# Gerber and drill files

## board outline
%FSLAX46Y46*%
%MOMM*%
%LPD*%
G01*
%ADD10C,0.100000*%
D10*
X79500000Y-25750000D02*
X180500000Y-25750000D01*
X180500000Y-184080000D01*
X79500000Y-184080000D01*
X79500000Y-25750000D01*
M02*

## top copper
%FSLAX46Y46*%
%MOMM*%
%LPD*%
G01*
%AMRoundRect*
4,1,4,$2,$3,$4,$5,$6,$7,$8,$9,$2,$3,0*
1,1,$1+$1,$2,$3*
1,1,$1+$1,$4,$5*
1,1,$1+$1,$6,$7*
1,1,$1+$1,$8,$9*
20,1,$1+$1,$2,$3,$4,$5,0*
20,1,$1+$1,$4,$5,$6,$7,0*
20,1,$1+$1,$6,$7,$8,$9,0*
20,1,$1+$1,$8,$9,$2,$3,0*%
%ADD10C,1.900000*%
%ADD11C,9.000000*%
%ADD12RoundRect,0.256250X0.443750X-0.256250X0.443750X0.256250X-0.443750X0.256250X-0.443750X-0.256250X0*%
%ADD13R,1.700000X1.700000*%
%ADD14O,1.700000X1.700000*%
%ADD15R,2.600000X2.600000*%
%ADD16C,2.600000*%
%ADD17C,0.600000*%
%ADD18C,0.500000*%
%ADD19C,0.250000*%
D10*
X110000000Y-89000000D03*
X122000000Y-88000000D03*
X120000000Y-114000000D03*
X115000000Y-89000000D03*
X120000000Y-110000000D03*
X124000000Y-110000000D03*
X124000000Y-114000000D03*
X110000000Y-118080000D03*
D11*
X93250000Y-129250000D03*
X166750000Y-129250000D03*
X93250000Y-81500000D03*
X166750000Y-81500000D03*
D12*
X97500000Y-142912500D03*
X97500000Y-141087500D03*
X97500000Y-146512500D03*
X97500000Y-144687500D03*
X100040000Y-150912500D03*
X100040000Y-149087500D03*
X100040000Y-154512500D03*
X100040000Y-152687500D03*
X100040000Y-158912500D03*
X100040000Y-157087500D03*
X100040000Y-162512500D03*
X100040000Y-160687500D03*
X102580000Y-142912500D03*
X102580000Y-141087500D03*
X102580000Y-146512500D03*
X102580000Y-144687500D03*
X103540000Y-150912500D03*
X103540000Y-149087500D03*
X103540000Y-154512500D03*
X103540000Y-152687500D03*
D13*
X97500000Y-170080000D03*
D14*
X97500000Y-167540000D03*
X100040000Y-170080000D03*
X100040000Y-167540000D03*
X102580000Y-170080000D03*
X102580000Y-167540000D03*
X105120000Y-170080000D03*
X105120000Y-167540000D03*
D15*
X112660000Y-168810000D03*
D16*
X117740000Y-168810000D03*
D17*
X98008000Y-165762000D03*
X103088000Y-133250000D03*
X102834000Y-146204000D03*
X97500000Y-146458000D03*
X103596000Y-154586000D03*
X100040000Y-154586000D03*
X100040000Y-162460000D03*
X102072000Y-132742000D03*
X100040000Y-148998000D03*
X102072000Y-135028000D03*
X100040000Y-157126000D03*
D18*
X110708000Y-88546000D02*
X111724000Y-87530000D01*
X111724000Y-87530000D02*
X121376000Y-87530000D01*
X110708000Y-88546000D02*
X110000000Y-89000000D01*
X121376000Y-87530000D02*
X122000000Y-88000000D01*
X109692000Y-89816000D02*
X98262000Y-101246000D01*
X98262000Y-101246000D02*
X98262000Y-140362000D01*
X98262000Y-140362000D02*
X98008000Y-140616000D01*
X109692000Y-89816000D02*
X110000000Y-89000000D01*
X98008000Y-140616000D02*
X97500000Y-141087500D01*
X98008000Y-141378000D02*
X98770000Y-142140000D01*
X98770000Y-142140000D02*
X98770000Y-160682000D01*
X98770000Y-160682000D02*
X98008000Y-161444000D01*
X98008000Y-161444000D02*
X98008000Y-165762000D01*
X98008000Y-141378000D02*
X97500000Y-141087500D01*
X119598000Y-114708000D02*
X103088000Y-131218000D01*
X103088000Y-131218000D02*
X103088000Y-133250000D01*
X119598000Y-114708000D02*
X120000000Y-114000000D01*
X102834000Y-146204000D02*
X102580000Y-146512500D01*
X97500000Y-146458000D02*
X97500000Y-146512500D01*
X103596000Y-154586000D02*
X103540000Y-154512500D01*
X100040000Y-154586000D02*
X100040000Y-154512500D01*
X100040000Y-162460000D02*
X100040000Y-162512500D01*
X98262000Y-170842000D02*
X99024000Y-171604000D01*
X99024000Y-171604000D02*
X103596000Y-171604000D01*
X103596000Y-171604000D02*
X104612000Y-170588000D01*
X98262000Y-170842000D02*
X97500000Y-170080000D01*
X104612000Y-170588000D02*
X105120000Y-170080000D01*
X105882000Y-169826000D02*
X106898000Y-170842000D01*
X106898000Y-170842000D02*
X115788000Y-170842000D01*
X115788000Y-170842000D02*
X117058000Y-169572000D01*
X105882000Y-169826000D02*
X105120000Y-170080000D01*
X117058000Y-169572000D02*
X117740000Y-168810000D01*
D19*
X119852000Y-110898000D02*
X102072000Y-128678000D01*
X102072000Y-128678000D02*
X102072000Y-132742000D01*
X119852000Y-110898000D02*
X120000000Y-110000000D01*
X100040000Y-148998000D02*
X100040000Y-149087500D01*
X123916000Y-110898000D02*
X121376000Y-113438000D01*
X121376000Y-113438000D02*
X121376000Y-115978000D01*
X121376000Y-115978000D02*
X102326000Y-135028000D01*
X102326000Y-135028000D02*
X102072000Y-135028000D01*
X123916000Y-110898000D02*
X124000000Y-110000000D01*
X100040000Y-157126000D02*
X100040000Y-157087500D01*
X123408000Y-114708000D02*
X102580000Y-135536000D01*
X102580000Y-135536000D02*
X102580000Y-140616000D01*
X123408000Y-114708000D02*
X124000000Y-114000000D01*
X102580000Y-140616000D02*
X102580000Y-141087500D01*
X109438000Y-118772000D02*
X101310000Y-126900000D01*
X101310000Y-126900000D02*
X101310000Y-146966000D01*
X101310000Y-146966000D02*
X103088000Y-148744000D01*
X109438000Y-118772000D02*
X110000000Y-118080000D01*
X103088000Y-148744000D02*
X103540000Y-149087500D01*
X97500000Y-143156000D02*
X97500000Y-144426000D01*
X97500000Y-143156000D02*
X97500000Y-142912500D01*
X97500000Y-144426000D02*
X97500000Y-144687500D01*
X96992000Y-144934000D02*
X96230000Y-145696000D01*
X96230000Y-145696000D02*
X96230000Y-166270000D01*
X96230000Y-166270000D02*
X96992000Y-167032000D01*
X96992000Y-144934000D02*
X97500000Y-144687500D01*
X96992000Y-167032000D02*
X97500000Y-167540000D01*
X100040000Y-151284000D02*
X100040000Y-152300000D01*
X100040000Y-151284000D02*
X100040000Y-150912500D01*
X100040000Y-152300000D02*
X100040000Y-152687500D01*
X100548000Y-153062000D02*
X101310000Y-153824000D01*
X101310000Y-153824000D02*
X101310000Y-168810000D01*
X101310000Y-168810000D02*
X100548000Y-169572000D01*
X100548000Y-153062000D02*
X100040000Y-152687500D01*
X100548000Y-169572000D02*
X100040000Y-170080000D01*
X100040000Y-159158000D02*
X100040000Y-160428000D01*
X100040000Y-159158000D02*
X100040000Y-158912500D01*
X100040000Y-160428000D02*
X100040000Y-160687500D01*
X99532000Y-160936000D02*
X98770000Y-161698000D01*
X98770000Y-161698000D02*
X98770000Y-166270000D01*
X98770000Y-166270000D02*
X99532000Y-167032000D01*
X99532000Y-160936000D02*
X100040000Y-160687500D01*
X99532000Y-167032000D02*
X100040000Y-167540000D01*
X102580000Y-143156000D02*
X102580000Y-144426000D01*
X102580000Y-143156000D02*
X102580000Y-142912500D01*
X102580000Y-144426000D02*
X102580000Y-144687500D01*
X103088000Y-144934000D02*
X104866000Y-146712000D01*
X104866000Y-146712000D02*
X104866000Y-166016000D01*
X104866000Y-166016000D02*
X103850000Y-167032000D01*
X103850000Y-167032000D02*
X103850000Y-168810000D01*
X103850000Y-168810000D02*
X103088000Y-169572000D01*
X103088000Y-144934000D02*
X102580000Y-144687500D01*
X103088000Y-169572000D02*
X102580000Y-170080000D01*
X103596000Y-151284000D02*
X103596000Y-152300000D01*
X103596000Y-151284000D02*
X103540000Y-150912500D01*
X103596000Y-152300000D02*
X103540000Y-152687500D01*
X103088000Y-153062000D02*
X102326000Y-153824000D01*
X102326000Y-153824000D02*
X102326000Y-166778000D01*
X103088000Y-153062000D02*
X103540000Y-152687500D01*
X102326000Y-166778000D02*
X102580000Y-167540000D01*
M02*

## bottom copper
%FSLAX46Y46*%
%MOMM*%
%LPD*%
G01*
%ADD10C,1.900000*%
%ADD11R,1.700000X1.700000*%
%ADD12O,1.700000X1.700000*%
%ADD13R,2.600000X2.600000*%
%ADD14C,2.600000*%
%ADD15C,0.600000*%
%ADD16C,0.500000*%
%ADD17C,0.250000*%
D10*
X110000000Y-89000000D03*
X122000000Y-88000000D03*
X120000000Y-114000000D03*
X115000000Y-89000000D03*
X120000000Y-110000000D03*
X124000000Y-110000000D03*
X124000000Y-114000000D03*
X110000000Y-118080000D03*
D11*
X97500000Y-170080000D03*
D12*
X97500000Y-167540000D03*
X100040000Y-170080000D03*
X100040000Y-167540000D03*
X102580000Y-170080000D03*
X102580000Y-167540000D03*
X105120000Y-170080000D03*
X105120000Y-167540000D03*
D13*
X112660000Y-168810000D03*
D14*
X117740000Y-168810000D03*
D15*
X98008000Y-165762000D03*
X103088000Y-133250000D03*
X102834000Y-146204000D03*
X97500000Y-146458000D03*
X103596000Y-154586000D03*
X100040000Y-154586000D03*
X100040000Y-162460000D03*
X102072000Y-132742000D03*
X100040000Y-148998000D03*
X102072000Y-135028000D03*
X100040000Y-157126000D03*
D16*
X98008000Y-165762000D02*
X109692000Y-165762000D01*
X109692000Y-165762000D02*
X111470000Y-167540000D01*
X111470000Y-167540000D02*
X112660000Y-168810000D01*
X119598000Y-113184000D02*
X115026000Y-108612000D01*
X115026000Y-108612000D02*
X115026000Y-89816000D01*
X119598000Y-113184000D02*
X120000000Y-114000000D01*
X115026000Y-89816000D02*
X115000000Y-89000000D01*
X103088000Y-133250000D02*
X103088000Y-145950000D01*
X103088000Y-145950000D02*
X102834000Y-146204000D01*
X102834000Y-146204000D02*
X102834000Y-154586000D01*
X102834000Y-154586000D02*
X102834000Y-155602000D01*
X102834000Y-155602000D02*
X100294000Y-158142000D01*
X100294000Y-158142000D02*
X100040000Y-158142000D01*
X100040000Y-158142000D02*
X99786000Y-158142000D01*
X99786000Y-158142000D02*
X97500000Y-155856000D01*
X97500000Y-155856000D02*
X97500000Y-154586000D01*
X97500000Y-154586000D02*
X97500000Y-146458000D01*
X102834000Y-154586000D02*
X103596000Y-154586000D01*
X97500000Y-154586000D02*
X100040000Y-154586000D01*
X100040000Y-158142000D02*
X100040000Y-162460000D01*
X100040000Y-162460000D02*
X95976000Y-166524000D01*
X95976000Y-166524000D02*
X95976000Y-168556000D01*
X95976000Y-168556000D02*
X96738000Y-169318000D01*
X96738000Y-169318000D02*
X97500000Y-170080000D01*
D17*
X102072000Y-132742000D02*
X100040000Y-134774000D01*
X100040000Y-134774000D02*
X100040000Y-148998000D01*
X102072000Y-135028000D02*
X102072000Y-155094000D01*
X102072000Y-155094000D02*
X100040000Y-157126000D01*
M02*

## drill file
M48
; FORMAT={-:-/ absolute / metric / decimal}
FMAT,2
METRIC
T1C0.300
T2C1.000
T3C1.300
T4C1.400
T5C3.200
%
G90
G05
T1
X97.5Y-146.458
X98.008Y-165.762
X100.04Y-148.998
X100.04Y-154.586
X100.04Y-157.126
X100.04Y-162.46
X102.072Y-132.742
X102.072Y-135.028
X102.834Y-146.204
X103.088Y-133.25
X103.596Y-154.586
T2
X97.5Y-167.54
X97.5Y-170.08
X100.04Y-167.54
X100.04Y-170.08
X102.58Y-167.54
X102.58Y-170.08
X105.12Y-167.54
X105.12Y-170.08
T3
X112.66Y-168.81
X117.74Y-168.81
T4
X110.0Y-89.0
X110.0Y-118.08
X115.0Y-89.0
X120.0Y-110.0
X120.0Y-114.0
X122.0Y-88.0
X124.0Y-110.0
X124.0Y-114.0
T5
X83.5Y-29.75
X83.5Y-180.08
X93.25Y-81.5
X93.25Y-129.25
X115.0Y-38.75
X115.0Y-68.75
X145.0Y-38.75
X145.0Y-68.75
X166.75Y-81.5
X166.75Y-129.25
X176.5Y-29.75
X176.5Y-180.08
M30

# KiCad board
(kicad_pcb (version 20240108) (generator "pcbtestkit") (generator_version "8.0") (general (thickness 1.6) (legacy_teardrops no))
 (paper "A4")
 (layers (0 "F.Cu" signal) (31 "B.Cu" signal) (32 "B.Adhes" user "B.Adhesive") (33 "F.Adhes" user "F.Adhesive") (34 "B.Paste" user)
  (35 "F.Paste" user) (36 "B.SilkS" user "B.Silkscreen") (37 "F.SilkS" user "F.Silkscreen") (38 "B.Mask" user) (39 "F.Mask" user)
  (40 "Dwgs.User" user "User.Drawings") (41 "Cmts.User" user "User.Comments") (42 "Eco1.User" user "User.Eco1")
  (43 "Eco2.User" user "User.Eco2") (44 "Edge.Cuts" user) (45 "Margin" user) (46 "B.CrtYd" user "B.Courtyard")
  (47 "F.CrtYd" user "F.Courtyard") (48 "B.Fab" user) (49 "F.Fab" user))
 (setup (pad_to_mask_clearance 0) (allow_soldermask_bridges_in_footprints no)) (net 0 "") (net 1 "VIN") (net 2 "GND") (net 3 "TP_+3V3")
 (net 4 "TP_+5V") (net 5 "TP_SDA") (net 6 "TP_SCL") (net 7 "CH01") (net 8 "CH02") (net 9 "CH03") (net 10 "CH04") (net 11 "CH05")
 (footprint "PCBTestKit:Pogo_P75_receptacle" (layer "F.Cu") (at 110 89)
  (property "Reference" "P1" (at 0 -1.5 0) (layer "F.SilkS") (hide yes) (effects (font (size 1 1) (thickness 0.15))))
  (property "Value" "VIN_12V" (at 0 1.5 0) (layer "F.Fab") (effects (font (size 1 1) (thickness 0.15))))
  (pad "1" thru_hole circle (at 0 0) (size 1.9 1.9) (drill 1.4) (layers "*.Cu" "*.Mask") (remove_unused_layers no) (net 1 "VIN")))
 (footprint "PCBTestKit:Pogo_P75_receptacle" (layer "F.Cu") (at 122 88)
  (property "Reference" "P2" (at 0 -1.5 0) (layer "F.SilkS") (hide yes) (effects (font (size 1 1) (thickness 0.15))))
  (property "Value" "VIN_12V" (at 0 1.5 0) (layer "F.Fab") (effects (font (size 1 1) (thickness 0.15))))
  (pad "1" thru_hole circle (at 0 0) (size 1.9 1.9) (drill 1.4) (layers "*.Cu" "*.Mask") (remove_unused_layers no) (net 1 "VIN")))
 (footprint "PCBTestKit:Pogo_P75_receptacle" (layer "F.Cu") (at 120 114)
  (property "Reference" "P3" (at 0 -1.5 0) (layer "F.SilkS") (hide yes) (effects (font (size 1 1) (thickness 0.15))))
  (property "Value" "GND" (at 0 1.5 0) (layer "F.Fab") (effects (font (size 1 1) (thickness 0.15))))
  (pad "1" thru_hole circle (at 0 0) (size 1.9 1.9) (drill 1.4) (layers "*.Cu" "*.Mask") (remove_unused_layers no) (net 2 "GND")))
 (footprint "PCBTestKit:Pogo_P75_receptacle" (layer "F.Cu") (at 115 89)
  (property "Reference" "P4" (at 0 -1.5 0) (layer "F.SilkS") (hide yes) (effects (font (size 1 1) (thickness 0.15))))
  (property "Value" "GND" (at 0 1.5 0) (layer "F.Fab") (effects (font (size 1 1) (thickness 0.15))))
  (pad "1" thru_hole circle (at 0 0) (size 1.9 1.9) (drill 1.4) (layers "*.Cu" "*.Mask") (remove_unused_layers no) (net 2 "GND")))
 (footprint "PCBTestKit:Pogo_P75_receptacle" (layer "F.Cu") (at 120 110)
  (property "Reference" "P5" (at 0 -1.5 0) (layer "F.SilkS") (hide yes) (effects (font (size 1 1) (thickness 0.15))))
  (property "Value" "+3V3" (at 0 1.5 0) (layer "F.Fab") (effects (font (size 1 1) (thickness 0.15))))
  (pad "1" thru_hole circle (at 0 0) (size 1.9 1.9) (drill 1.4) (layers "*.Cu" "*.Mask") (remove_unused_layers no) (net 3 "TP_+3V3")))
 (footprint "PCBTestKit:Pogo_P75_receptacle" (layer "F.Cu") (at 124 110)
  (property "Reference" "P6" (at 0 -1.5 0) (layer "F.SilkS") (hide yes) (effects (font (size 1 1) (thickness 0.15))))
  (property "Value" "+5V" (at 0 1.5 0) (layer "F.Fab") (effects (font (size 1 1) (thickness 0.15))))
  (pad "1" thru_hole circle (at 0 0) (size 1.9 1.9) (drill 1.4) (layers "*.Cu" "*.Mask") (remove_unused_layers no) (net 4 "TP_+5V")))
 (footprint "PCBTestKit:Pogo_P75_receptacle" (layer "F.Cu") (at 124 114)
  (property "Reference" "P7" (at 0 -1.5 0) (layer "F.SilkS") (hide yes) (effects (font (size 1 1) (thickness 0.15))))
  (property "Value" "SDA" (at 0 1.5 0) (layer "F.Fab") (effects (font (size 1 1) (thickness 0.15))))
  (pad "1" thru_hole circle (at 0 0) (size 1.9 1.9) (drill 1.4) (layers "*.Cu" "*.Mask") (remove_unused_layers no) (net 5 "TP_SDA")))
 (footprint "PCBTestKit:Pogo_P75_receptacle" (layer "F.Cu") (at 110 118.08)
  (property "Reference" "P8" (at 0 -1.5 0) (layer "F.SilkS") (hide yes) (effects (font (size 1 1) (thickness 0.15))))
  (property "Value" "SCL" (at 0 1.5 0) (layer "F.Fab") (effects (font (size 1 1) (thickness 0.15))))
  (pad "1" thru_hole circle (at 0 0) (size 1.9 1.9) (drill 1.4) (layers "*.Cu" "*.Mask") (remove_unused_layers no) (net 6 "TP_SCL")))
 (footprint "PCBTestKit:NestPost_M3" (layer "F.Cu") (at 93.25 129.25)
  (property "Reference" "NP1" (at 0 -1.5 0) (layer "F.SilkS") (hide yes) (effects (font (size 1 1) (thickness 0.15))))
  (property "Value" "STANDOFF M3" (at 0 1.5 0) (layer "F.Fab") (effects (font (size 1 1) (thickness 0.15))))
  (pad "" np_thru_hole circle (at 0 0) (size 9 9) (drill 3.2) (layers "F.Cu" "F.Mask")))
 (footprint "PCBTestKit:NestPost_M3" (layer "F.Cu") (at 166.75 129.25)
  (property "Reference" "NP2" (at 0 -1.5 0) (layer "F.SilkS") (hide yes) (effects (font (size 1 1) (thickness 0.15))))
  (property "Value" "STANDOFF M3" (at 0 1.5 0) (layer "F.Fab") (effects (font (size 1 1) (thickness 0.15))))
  (pad "" np_thru_hole circle (at 0 0) (size 9 9) (drill 3.2) (layers "F.Cu" "F.Mask")))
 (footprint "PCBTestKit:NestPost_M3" (layer "F.Cu") (at 93.25 81.5)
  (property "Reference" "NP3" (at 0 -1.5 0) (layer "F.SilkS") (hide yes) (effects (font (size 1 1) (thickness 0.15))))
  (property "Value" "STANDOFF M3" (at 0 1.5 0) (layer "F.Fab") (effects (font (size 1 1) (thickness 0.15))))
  (pad "" np_thru_hole circle (at 0 0) (size 9 9) (drill 3.2) (layers "F.Cu" "F.Mask")))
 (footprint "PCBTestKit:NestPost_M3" (layer "F.Cu") (at 166.75 81.5)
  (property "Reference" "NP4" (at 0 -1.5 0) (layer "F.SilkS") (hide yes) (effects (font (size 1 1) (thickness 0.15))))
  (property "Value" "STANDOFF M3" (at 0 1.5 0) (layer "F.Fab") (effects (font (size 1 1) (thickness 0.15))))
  (pad "" np_thru_hole circle (at 0 0) (size 9 9) (drill 3.2) (layers "F.Cu" "F.Mask")))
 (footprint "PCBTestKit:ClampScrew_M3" (layer "F.Cu") (at 115 68.75)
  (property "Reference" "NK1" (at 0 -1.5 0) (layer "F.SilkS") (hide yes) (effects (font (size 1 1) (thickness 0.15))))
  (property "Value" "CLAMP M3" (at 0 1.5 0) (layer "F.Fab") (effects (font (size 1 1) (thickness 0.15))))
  (pad "" np_thru_hole circle (at 0 0) (size 3.2 3.2) (drill 3.2) (layers "*.Cu" "*.Mask")))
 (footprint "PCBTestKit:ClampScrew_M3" (layer "F.Cu") (at 115 38.75)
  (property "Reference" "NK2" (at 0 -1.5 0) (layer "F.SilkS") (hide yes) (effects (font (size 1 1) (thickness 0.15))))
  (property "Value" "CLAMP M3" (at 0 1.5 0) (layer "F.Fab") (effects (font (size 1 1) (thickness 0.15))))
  (pad "" np_thru_hole circle (at 0 0) (size 3.2 3.2) (drill 3.2) (layers "*.Cu" "*.Mask")))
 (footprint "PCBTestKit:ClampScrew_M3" (layer "F.Cu") (at 145 68.75)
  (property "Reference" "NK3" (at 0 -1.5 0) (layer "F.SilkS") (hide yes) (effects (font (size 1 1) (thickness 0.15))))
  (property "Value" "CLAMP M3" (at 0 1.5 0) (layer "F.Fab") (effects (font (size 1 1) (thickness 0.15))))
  (pad "" np_thru_hole circle (at 0 0) (size 3.2 3.2) (drill 3.2) (layers "*.Cu" "*.Mask")))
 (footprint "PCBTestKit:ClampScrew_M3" (layer "F.Cu") (at 145 38.75)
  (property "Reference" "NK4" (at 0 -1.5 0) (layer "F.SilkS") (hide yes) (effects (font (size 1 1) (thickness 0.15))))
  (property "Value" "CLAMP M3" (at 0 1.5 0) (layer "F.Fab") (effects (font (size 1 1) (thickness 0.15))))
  (pad "" np_thru_hole circle (at 0 0) (size 3.2 3.2) (drill 3.2) (layers "*.Cu" "*.Mask")))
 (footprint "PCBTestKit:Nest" (layer "F.Cu") (at 130 102.5)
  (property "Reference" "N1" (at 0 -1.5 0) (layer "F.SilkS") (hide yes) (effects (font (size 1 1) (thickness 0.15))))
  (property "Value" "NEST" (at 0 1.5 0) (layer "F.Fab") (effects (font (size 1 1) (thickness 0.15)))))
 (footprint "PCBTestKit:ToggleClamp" (layer "F.Cu") (at 130 102.5)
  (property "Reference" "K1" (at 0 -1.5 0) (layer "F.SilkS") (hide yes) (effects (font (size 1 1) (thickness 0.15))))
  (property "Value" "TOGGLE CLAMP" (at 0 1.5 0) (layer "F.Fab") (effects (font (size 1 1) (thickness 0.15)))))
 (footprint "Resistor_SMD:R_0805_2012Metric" (layer "F.Cu") (at 97.5 142 90)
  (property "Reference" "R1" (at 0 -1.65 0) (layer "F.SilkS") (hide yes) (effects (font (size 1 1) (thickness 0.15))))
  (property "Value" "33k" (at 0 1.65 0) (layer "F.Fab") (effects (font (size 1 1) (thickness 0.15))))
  (pad "1" smd roundrect (at -0.9125 0 90) (size 1.025 1.4) (layers "F.Cu" "F.Paste" "F.Mask") (roundrect_rratio 0.25) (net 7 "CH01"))
  (pad "2" smd roundrect (at 0.9125 0 90) (size 1.025 1.4) (layers "F.Cu" "F.Paste" "F.Mask") (roundrect_rratio 0.25) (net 1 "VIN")))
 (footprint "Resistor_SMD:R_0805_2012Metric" (layer "F.Cu") (at 97.5 145.6 90)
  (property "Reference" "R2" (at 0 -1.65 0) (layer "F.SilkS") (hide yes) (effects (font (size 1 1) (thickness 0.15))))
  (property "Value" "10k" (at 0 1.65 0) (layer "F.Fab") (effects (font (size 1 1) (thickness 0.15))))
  (pad "1" smd roundrect (at -0.9125 0 90) (size 1.025 1.4) (layers "F.Cu" "F.Paste" "F.Mask") (roundrect_rratio 0.25) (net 2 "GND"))
  (pad "2" smd roundrect (at 0.9125 0 90) (size 1.025 1.4) (layers "F.Cu" "F.Paste" "F.Mask") (roundrect_rratio 0.25) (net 7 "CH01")))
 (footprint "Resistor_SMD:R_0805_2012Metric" (layer "F.Cu") (at 100.04 150 90)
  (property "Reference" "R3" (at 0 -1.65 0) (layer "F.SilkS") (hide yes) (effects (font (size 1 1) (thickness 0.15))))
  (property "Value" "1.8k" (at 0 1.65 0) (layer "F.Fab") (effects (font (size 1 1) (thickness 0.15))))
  (pad "1" smd roundrect (at -0.9125 0 90) (size 1.025 1.4) (layers "F.Cu" "F.Paste" "F.Mask") (roundrect_rratio 0.25) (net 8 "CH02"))
  (pad "2" smd roundrect (at 0.9125 0 90) (size 1.025 1.4) (layers "F.Cu" "F.Paste" "F.Mask") (roundrect_rratio 0.25) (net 3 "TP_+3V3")))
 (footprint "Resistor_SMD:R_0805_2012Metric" (layer "F.Cu") (at 100.04 153.6 90)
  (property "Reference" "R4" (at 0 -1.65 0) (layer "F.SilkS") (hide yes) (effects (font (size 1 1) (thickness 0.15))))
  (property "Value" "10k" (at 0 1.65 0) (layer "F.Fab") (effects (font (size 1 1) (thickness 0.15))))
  (pad "1" smd roundrect (at -0.9125 0 90) (size 1.025 1.4) (layers "F.Cu" "F.Paste" "F.Mask") (roundrect_rratio 0.25) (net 2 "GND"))
  (pad "2" smd roundrect (at 0.9125 0 90) (size 1.025 1.4) (layers "F.Cu" "F.Paste" "F.Mask") (roundrect_rratio 0.25) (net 8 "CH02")))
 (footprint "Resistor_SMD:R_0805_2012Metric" (layer "F.Cu") (at 100.04 158 90)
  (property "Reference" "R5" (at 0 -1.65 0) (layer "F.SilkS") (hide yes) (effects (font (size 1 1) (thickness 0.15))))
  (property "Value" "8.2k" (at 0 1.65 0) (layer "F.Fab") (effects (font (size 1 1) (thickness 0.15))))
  (pad "1" smd roundrect (at -0.9125 0 90) (size 1.025 1.4) (layers "F.Cu" "F.Paste" "F.Mask") (roundrect_rratio 0.25) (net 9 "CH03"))
  (pad "2" smd roundrect (at 0.9125 0 90) (size 1.025 1.4) (layers "F.Cu" "F.Paste" "F.Mask") (roundrect_rratio 0.25) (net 4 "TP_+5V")))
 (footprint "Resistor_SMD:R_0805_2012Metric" (layer "F.Cu") (at 100.04 161.6 90)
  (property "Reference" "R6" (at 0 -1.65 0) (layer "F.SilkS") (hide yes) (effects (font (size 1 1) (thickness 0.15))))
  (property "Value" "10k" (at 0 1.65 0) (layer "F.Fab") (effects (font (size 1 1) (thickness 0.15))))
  (pad "1" smd roundrect (at -0.9125 0 90) (size 1.025 1.4) (layers "F.Cu" "F.Paste" "F.Mask") (roundrect_rratio 0.25) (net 2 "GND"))
  (pad "2" smd roundrect (at 0.9125 0 90) (size 1.025 1.4) (layers "F.Cu" "F.Paste" "F.Mask") (roundrect_rratio 0.25) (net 9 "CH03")))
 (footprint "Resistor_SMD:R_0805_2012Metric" (layer "F.Cu") (at 102.58 142 90)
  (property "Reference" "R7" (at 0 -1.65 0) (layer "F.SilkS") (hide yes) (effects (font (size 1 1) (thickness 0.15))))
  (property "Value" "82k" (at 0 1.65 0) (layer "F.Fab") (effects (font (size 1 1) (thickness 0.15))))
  (pad "1" smd roundrect (at -0.9125 0 90) (size 1.025 1.4) (layers "F.Cu" "F.Paste" "F.Mask") (roundrect_rratio 0.25) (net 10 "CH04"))
  (pad "2" smd roundrect (at 0.9125 0 90) (size 1.025 1.4) (layers "F.Cu" "F.Paste" "F.Mask") (roundrect_rratio 0.25) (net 5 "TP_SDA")))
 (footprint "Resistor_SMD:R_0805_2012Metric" (layer "F.Cu") (at 102.58 145.6 90)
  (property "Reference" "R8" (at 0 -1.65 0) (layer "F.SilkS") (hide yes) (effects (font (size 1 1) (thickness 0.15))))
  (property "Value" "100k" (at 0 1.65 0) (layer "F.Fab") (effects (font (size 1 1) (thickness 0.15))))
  (pad "1" smd roundrect (at -0.9125 0 90) (size 1.025 1.4) (layers "F.Cu" "F.Paste" "F.Mask") (roundrect_rratio 0.25) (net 2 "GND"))
  (pad "2" smd roundrect (at 0.9125 0 90) (size 1.025 1.4) (layers "F.Cu" "F.Paste" "F.Mask") (roundrect_rratio 0.25) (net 10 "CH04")))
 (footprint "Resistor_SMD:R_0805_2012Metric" (layer "F.Cu") (at 103.54 150 90)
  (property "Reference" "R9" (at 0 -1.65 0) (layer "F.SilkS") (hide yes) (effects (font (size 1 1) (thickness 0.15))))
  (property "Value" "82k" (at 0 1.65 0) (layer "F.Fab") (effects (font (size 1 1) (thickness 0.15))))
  (pad "1" smd roundrect (at -0.9125 0 90) (size 1.025 1.4) (layers "F.Cu" "F.Paste" "F.Mask") (roundrect_rratio 0.25) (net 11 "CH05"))
  (pad "2" smd roundrect (at 0.9125 0 90) (size 1.025 1.4) (layers "F.Cu" "F.Paste" "F.Mask") (roundrect_rratio 0.25) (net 6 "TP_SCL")))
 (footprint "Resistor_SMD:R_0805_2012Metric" (layer "F.Cu") (at 103.54 153.6 90)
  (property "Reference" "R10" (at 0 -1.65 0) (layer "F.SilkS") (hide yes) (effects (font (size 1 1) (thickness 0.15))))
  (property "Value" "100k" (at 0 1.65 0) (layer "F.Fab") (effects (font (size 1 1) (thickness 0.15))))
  (pad "1" smd roundrect (at -0.9125 0 90) (size 1.025 1.4) (layers "F.Cu" "F.Paste" "F.Mask") (roundrect_rratio 0.25) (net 2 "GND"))
  (pad "2" smd roundrect (at 0.9125 0 90) (size 1.025 1.4) (layers "F.Cu" "F.Paste" "F.Mask") (roundrect_rratio 0.25) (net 11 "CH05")))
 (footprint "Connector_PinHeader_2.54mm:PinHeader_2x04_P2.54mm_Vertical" (layer "F.Cu") (at 97.5 170.08 90)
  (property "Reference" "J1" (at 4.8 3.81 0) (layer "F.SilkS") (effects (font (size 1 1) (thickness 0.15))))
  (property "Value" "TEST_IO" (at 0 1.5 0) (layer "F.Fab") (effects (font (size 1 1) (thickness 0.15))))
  (pad "1" thru_hole rect (at 0 0 90) (size 1.7 1.7) (drill 1) (layers "*.Cu" "*.Mask") (remove_unused_layers no) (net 2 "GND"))
  (pad "2" thru_hole oval (at 2.54 0 90) (size 1.7 1.7) (drill 1) (layers "*.Cu" "*.Mask") (remove_unused_layers no) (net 7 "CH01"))
  (pad "3" thru_hole oval (at 0 2.54 90) (size 1.7 1.7) (drill 1) (layers "*.Cu" "*.Mask") (remove_unused_layers no) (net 8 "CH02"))
  (pad "4" thru_hole oval (at 2.54 2.54 90) (size 1.7 1.7) (drill 1) (layers "*.Cu" "*.Mask") (remove_unused_layers no) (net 9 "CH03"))
  (pad "5" thru_hole oval (at 0 5.08 90) (size 1.7 1.7) (drill 1) (layers "*.Cu" "*.Mask") (remove_unused_layers no) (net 10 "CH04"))
  (pad "6" thru_hole oval (at 2.54 5.08 90) (size 1.7 1.7) (drill 1) (layers "*.Cu" "*.Mask") (remove_unused_layers no) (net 11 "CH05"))
  (pad "7" thru_hole oval (at 0 7.62 90) (size 1.7 1.7) (drill 1) (layers "*.Cu" "*.Mask") (remove_unused_layers no) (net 2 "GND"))
  (pad "8" thru_hole oval (at 2.54 7.62 90) (size 1.7 1.7) (drill 1) (layers "*.Cu" "*.Mask") (remove_unused_layers no)))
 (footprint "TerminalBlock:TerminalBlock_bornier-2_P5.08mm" (layer "F.Cu") (at 112.66 168.81)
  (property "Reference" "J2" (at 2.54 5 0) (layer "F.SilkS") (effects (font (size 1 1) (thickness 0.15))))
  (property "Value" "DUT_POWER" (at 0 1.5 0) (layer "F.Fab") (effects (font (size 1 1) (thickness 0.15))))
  (pad "1" thru_hole rect (at 0 0) (size 2.6 2.6) (drill 1.3) (layers "*.Cu" "*.Mask") (remove_unused_layers no) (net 1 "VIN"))
  (pad "2" thru_hole circle (at 5.08 0) (size 2.6 2.6) (drill 1.3) (layers "*.Cu" "*.Mask") (remove_unused_layers no) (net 2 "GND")))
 (gr_rect (start 79.5 25.75) (end 180.5 184.08) (stroke (width 0.1) (type solid)) (fill none) (layer "Edge.Cuts"))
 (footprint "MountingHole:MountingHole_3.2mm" (layer "F.Cu") (at 83.5 29.75)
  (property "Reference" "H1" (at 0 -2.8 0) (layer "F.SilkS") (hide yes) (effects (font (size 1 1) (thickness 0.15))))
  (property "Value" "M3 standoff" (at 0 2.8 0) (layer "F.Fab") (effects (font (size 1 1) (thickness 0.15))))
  (pad "" np_thru_hole circle (at 0 0) (size 3.2 3.2) (drill 3.2) (layers "*.Cu" "*.Mask")))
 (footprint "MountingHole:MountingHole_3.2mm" (layer "F.Cu") (at 176.5 29.75)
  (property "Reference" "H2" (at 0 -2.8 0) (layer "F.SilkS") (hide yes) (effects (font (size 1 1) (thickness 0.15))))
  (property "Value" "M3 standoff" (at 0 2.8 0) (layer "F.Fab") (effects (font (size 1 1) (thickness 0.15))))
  (pad "" np_thru_hole circle (at 0 0) (size 3.2 3.2) (drill 3.2) (layers "*.Cu" "*.Mask")))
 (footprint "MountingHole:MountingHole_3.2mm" (layer "F.Cu") (at 83.5 180.08)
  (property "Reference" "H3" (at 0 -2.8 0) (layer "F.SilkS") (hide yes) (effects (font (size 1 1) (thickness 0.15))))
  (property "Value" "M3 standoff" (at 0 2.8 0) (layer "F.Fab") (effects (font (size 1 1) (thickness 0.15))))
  (pad "" np_thru_hole circle (at 0 0) (size 3.2 3.2) (drill 3.2) (layers "*.Cu" "*.Mask")))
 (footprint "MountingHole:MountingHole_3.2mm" (layer "F.Cu") (at 176.5 180.08)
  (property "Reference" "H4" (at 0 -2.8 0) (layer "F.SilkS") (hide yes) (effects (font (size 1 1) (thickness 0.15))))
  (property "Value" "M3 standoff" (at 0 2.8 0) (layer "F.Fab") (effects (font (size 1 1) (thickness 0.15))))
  (pad "" np_thru_hole circle (at 0 0) (size 3.2 3.2) (drill 3.2) (layers "*.Cu" "*.Mask")))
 (segment (start 110.708 88.546) (end 111.724 87.53) (width 0.5) (layer "F.Cu") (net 1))
 (segment (start 111.724 87.53) (end 121.376 87.53) (width 0.5) (layer "F.Cu") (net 1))
 (segment (start 110.708 88.546) (end 110 89) (width 0.5) (layer "F.Cu") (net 1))
 (segment (start 121.376 87.53) (end 122 88) (width 0.5) (layer "F.Cu") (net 1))
 (segment (start 109.692 89.816) (end 98.262 101.246) (width 0.5) (layer "F.Cu") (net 1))
 (segment (start 98.262 101.246) (end 98.262 140.362) (width 0.5) (layer "F.Cu") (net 1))
 (segment (start 98.262 140.362) (end 98.008 140.616) (width 0.5) (layer "F.Cu") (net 1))
 (segment (start 109.692 89.816) (end 110 89) (width 0.5) (layer "F.Cu") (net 1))
 (segment (start 98.008 140.616) (end 97.5 141.0875) (width 0.5) (layer "F.Cu") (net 1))
 (segment (start 98.008 141.378) (end 98.77 142.14) (width 0.5) (layer "F.Cu") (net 1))
 (segment (start 98.77 142.14) (end 98.77 160.682) (width 0.5) (layer "F.Cu") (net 1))
 (segment (start 98.77 160.682) (end 98.008 161.444) (width 0.5) (layer "F.Cu") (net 1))
 (segment (start 98.008 161.444) (end 98.008 165.762) (width 0.5) (layer "F.Cu") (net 1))
 (segment (start 98.008 165.762) (end 109.692 165.762) (width 0.5) (layer "B.Cu") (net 1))
 (segment (start 109.692 165.762) (end 111.47 167.54) (width 0.5) (layer "B.Cu") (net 1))
 (segment (start 98.008 141.378) (end 97.5 141.0875) (width 0.5) (layer "F.Cu") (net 1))
 (segment (start 111.47 167.54) (end 112.66 168.81) (width 0.5) (layer "B.Cu") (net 1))
 (segment (start 119.598 113.184) (end 115.026 108.612) (width 0.5) (layer "B.Cu") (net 2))
 (segment (start 115.026 108.612) (end 115.026 89.816) (width 0.5) (layer "B.Cu") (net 2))
 (segment (start 119.598 113.184) (end 120 114) (width 0.5) (layer "B.Cu") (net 2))
 (segment (start 115.026 89.816) (end 115 89) (width 0.5) (layer "B.Cu") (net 2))
 (segment (start 119.598 114.708) (end 103.088 131.218) (width 0.5) (layer "F.Cu") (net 2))
 (segment (start 103.088 131.218) (end 103.088 133.25) (width 0.5) (layer "F.Cu") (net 2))
 (segment (start 103.088 133.25) (end 103.088 145.95) (width 0.5) (layer "B.Cu") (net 2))
 (segment (start 103.088 145.95) (end 102.834 146.204) (width 0.5) (layer "B.Cu") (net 2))
 (segment (start 119.598 114.708) (end 120 114) (width 0.5) (layer "F.Cu") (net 2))
 (segment (start 102.834 146.204) (end 102.58 146.5125) (width 0.5) (layer "F.Cu") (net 2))
 (segment (start 102.834 146.204) (end 102.834 154.586) (width 0.5) (layer "B.Cu") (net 2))
 (segment (start 102.834 154.586) (end 102.834 155.602) (width 0.5) (layer "B.Cu") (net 2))
 (segment (start 102.834 155.602) (end 100.294 158.142) (width 0.5) (layer "B.Cu") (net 2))
 (segment (start 100.294 158.142) (end 100.04 158.142) (width 0.5) (layer "B.Cu") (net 2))
 (segment (start 100.04 158.142) (end 99.786 158.142) (width 0.5) (layer "B.Cu") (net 2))
 (segment (start 99.786 158.142) (end 97.5 155.856) (width 0.5) (layer "B.Cu") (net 2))
 (segment (start 97.5 155.856) (end 97.5 154.586) (width 0.5) (layer "B.Cu") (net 2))
 (segment (start 97.5 154.586) (end 97.5 146.458) (width 0.5) (layer "B.Cu") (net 2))
 (segment (start 97.5 146.458) (end 97.5 146.5125) (width 0.5) (layer "F.Cu") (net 2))
 (segment (start 102.834 154.586) (end 103.596 154.586) (width 0.5) (layer "B.Cu") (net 2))
 (segment (start 103.596 154.586) (end 103.54 154.5125) (width 0.5) (layer "F.Cu") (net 2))
 (segment (start 97.5 154.586) (end 100.04 154.586) (width 0.5) (layer "B.Cu") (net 2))
 (segment (start 100.04 154.586) (end 100.04 154.5125) (width 0.5) (layer "F.Cu") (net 2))
 (segment (start 100.04 158.142) (end 100.04 162.46) (width 0.5) (layer "B.Cu") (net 2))
 (segment (start 100.04 162.46) (end 100.04 162.5125) (width 0.5) (layer "F.Cu") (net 2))
 (segment (start 100.04 162.46) (end 95.976 166.524) (width 0.5) (layer "B.Cu") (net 2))
 (segment (start 95.976 166.524) (end 95.976 168.556) (width 0.5) (layer "B.Cu") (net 2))
 (segment (start 95.976 168.556) (end 96.738 169.318) (width 0.5) (layer "B.Cu") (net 2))
 (segment (start 96.738 169.318) (end 97.5 170.08) (width 0.5) (layer "B.Cu") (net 2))
 (segment (start 98.262 170.842) (end 99.024 171.604) (width 0.5) (layer "F.Cu") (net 2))
 (segment (start 99.024 171.604) (end 103.596 171.604) (width 0.5) (layer "F.Cu") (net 2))
 (segment (start 103.596 171.604) (end 104.612 170.588) (width 0.5) (layer "F.Cu") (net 2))
 (segment (start 98.262 170.842) (end 97.5 170.08) (width 0.5) (layer "F.Cu") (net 2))
 (segment (start 104.612 170.588) (end 105.12 170.08) (width 0.5) (layer "F.Cu") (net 2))
 (segment (start 105.882 169.826) (end 106.898 170.842) (width 0.5) (layer "F.Cu") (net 2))
 (segment (start 106.898 170.842) (end 115.788 170.842) (width 0.5) (layer "F.Cu") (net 2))
 (segment (start 115.788 170.842) (end 117.058 169.572) (width 0.5) (layer "F.Cu") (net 2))
 (segment (start 105.882 169.826) (end 105.12 170.08) (width 0.5) (layer "F.Cu") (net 2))
 (segment (start 117.058 169.572) (end 117.74 168.81) (width 0.5) (layer "F.Cu") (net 2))
 (segment (start 119.852 110.898) (end 102.072 128.678) (width 0.25) (layer "F.Cu") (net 3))
 (segment (start 102.072 128.678) (end 102.072 132.742) (width 0.25) (layer "F.Cu") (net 3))
 (segment (start 102.072 132.742) (end 100.04 134.774) (width 0.25) (layer "B.Cu") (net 3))
 (segment (start 100.04 134.774) (end 100.04 148.998) (width 0.25) (layer "B.Cu") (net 3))
 (segment (start 119.852 110.898) (end 120 110) (width 0.25) (layer "F.Cu") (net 3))
 (segment (start 100.04 148.998) (end 100.04 149.0875) (width 0.25) (layer "F.Cu") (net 3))
 (segment (start 123.916 110.898) (end 121.376 113.438) (width 0.25) (layer "F.Cu") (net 4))
 (segment (start 121.376 113.438) (end 121.376 115.978) (width 0.25) (layer "F.Cu") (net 4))
 (segment (start 121.376 115.978) (end 102.326 135.028) (width 0.25) (layer "F.Cu") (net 4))
 (segment (start 102.326 135.028) (end 102.072 135.028) (width 0.25) (layer "F.Cu") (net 4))
 (segment (start 102.072 135.028) (end 102.072 155.094) (width 0.25) (layer "B.Cu") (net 4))
 (segment (start 102.072 155.094) (end 100.04 157.126) (width 0.25) (layer "B.Cu") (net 4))
 (segment (start 123.916 110.898) (end 124 110) (width 0.25) (layer "F.Cu") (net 4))
 (segment (start 100.04 157.126) (end 100.04 157.0875) (width 0.25) (layer "F.Cu") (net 4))
 (segment (start 123.408 114.708) (end 102.58 135.536) (width 0.25) (layer "F.Cu") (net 5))
 (segment (start 102.58 135.536) (end 102.58 140.616) (width 0.25) (layer "F.Cu") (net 5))
 (segment (start 123.408 114.708) (end 124 114) (width 0.25) (layer "F.Cu") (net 5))
 (segment (start 102.58 140.616) (end 102.58 141.0875) (width 0.25) (layer "F.Cu") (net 5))
 (segment (start 109.438 118.772) (end 101.31 126.9) (width 0.25) (layer "F.Cu") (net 6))
 (segment (start 101.31 126.9) (end 101.31 146.966) (width 0.25) (layer "F.Cu") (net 6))
 (segment (start 101.31 146.966) (end 103.088 148.744) (width 0.25) (layer "F.Cu") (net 6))
 (segment (start 109.438 118.772) (end 110 118.08) (width 0.25) (layer "F.Cu") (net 6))
 (segment (start 103.088 148.744) (end 103.54 149.0875) (width 0.25) (layer "F.Cu") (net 6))
 (segment (start 97.5 143.156) (end 97.5 144.426) (width 0.25) (layer "F.Cu") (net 7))
 (segment (start 97.5 143.156) (end 97.5 142.9125) (width 0.25) (layer "F.Cu") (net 7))
 (segment (start 97.5 144.426) (end 97.5 144.6875) (width 0.25) (layer "F.Cu") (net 7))
 (segment (start 96.992 144.934) (end 96.23 145.696) (width 0.25) (layer "F.Cu") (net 7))
 (segment (start 96.23 145.696) (end 96.23 166.27) (width 0.25) (layer "F.Cu") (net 7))
 (segment (start 96.23 166.27) (end 96.992 167.032) (width 0.25) (layer "F.Cu") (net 7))
 (segment (start 96.992 144.934) (end 97.5 144.6875) (width 0.25) (layer "F.Cu") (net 7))
 (segment (start 96.992 167.032) (end 97.5 167.54) (width 0.25) (layer "F.Cu") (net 7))
 (segment (start 100.04 151.284) (end 100.04 152.3) (width 0.25) (layer "F.Cu") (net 8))
 (segment (start 100.04 151.284) (end 100.04 150.9125) (width 0.25) (layer "F.Cu") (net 8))
 (segment (start 100.04 152.3) (end 100.04 152.6875) (width 0.25) (layer "F.Cu") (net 8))
 (segment (start 100.548 153.062) (end 101.31 153.824) (width 0.25) (layer "F.Cu") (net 8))
 (segment (start 101.31 153.824) (end 101.31 168.81) (width 0.25) (layer "F.Cu") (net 8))
 (segment (start 101.31 168.81) (end 100.548 169.572) (width 0.25) (layer "F.Cu") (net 8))
 (segment (start 100.548 153.062) (end 100.04 152.6875) (width 0.25) (layer "F.Cu") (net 8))
 (segment (start 100.548 169.572) (end 100.04 170.08) (width 0.25) (layer "F.Cu") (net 8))
 (segment (start 100.04 159.158) (end 100.04 160.428) (width 0.25) (layer "F.Cu") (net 9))
 (segment (start 100.04 159.158) (end 100.04 158.9125) (width 0.25) (layer "F.Cu") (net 9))
 (segment (start 100.04 160.428) (end 100.04 160.6875) (width 0.25) (layer "F.Cu") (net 9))
 (segment (start 99.532 160.936) (end 98.77 161.698) (width 0.25) (layer "F.Cu") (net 9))
 (segment (start 98.77 161.698) (end 98.77 166.27) (width 0.25) (layer "F.Cu") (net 9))
 (segment (start 98.77 166.27) (end 99.532 167.032) (width 0.25) (layer "F.Cu") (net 9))
 (segment (start 99.532 160.936) (end 100.04 160.6875) (width 0.25) (layer "F.Cu") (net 9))
 (segment (start 99.532 167.032) (end 100.04 167.54) (width 0.25) (layer "F.Cu") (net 9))
 (segment (start 102.58 143.156) (end 102.58 144.426) (width 0.25) (layer "F.Cu") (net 10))
 (segment (start 102.58 143.156) (end 102.58 142.9125) (width 0.25) (layer "F.Cu") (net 10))
 (segment (start 102.58 144.426) (end 102.58 144.6875) (width 0.25) (layer "F.Cu") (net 10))
 (segment (start 103.088 144.934) (end 104.866 146.712) (width 0.25) (layer "F.Cu") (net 10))
 (segment (start 104.866 146.712) (end 104.866 166.016) (width 0.25) (layer "F.Cu") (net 10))
 (segment (start 104.866 166.016) (end 103.85 167.032) (width 0.25) (layer "F.Cu") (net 10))
 (segment (start 103.85 167.032) (end 103.85 168.81) (width 0.25) (layer "F.Cu") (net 10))
 (segment (start 103.85 168.81) (end 103.088 169.572) (width 0.25) (layer "F.Cu") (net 10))
 (segment (start 103.088 144.934) (end 102.58 144.6875) (width 0.25) (layer "F.Cu") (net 10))
 (segment (start 103.088 169.572) (end 102.58 170.08) (width 0.25) (layer "F.Cu") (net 10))
 (segment (start 103.596 151.284) (end 103.596 152.3) (width 0.25) (layer "F.Cu") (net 11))
 (segment (start 103.596 151.284) (end 103.54 150.9125) (width 0.25) (layer "F.Cu") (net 11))
 (segment (start 103.596 152.3) (end 103.54 152.6875) (width 0.25) (layer "F.Cu") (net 11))
 (segment (start 103.088 153.062) (end 102.326 153.824) (width 0.25) (layer "F.Cu") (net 11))
 (segment (start 102.326 153.824) (end 102.326 166.778) (width 0.25) (layer "F.Cu") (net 11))
 (segment (start 103.088 153.062) (end 103.54 152.6875) (width 0.25) (layer "F.Cu") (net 11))
 (segment (start 102.326 166.778) (end 102.58 167.54) (width 0.25) (layer "F.Cu") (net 11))
 (via (at 98.008 165.762) (size 0.6) (drill 0.3) (layers "F.Cu" "B.Cu") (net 1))
 (via (at 103.088 133.25) (size 0.6) (drill 0.3) (layers "F.Cu" "B.Cu") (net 2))
 (via (at 102.834 146.204) (size 0.6) (drill 0.3) (layers "F.Cu" "B.Cu") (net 2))
 (via (at 97.5 146.458) (size 0.6) (drill 0.3) (layers "F.Cu" "B.Cu") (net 2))
 (via (at 103.596 154.586) (size 0.6) (drill 0.3) (layers "F.Cu" "B.Cu") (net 2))
 (via (at 100.04 154.586) (size 0.6) (drill 0.3) (layers "F.Cu" "B.Cu") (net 2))
 (via (at 100.04 162.46) (size 0.6) (drill 0.3) (layers "F.Cu" "B.Cu") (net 2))
 (via (at 102.072 132.742) (size 0.6) (drill 0.3) (layers "F.Cu" "B.Cu") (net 3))
 (via (at 100.04 148.998) (size 0.6) (drill 0.3) (layers "F.Cu" "B.Cu") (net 3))
 (via (at 102.072 135.028) (size 0.6) (drill 0.3) (layers "F.Cu" "B.Cu") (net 4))
 (via (at 100.04 157.126) (size 0.6) (drill 0.3) (layers "F.Cu" "B.Cu") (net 4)))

